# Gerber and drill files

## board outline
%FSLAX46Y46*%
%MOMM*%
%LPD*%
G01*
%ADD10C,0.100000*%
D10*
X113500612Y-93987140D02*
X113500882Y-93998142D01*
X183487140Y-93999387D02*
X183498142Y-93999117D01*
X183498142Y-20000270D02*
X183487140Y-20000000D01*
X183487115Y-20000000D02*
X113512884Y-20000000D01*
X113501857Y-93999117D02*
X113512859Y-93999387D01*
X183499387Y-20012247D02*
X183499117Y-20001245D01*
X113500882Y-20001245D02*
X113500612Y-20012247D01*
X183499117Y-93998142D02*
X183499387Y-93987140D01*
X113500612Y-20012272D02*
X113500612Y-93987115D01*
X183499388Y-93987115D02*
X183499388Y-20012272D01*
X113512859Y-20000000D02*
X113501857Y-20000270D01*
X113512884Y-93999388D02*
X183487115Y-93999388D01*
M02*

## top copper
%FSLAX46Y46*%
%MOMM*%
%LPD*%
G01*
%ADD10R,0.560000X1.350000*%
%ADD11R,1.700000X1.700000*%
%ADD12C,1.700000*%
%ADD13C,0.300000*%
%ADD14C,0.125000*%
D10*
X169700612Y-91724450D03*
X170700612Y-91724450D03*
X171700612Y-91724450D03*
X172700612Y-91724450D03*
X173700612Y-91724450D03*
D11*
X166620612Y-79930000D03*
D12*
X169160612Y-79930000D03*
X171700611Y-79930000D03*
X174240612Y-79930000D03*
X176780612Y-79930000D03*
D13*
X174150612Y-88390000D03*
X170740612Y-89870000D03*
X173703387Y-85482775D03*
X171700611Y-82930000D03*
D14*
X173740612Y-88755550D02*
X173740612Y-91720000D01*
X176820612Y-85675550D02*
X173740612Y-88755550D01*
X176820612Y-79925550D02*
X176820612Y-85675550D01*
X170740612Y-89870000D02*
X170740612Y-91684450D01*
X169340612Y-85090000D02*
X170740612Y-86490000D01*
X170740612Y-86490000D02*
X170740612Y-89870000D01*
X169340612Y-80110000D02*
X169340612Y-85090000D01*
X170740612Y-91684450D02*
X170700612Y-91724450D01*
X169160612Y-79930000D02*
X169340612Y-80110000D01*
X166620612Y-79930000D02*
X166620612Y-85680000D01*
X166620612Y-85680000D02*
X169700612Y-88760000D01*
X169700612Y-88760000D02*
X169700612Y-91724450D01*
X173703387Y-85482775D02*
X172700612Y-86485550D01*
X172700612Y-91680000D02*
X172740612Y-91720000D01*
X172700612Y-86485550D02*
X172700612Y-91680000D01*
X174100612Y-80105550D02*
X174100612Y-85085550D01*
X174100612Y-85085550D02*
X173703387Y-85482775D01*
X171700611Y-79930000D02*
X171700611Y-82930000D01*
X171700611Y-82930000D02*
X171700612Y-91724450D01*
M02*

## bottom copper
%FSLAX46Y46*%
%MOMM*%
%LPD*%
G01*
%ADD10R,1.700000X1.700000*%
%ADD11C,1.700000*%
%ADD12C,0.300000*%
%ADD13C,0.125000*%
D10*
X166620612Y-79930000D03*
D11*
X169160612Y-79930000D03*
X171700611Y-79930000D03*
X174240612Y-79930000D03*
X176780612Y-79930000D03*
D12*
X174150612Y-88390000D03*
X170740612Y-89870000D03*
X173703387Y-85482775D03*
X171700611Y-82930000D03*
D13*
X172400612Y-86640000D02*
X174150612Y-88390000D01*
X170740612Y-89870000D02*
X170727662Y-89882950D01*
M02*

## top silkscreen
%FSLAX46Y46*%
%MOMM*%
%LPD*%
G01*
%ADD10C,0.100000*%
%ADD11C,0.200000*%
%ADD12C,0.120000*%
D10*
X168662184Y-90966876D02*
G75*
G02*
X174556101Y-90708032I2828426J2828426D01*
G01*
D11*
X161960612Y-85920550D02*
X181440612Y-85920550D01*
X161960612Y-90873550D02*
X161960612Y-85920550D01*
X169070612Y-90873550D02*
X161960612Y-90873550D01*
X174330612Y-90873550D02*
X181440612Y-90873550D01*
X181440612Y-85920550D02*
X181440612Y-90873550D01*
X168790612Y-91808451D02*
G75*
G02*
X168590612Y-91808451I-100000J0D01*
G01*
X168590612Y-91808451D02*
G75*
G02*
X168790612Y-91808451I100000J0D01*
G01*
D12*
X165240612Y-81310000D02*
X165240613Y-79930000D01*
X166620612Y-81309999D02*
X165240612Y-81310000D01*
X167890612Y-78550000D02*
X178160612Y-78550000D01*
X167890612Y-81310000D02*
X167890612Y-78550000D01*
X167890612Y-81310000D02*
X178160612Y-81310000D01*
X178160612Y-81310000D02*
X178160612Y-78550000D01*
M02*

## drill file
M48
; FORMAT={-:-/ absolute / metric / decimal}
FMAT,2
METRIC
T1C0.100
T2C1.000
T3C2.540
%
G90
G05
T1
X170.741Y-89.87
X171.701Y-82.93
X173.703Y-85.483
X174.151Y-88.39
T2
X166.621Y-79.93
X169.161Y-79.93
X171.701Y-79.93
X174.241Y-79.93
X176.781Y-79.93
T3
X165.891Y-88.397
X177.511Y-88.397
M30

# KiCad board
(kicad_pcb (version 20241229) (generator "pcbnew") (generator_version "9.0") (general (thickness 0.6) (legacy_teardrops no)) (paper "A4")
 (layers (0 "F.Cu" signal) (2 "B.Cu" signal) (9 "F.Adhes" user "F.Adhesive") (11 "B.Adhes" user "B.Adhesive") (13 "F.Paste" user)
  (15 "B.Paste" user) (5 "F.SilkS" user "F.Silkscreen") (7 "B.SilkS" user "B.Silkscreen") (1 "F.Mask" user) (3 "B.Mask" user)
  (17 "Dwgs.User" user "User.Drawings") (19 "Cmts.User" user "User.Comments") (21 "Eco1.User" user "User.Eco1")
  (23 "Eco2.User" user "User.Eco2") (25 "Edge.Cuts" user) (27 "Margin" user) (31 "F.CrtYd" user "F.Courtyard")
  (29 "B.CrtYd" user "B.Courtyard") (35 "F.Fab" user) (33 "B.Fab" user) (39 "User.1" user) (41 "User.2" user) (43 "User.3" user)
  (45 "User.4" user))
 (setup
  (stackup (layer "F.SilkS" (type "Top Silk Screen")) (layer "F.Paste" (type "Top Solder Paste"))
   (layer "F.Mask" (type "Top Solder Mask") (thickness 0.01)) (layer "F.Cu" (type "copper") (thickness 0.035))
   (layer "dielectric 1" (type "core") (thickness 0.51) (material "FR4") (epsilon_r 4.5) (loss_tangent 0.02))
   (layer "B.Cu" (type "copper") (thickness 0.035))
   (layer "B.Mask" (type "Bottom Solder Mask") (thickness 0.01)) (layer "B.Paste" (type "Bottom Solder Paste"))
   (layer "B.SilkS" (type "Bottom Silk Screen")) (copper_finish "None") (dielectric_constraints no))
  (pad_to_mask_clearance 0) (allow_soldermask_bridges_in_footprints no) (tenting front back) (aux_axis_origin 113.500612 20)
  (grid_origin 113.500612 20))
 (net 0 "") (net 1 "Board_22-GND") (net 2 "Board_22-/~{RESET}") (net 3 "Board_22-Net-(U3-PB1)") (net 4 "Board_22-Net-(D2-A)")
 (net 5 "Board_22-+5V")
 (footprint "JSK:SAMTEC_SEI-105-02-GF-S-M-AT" (layer "F.Cu") (at 171.700612 88.39845)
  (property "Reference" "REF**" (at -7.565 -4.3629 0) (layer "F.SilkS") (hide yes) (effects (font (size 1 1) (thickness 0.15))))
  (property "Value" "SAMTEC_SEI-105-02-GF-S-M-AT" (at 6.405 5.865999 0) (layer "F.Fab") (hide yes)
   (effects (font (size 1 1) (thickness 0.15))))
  (fp_line (start -9.74 -2.4779) (end 9.74 -2.4779) (stroke (width 0.2) (type solid)) (layer "F.SilkS"))
  (fp_line (start -9.74 2.4751) (end -9.74 -2.4779) (stroke (width 0.2) (type solid)) (layer "F.SilkS"))
  (fp_line (start -2.63 2.4751) (end -9.74 2.4751) (stroke (width 0.2) (type solid)) (layer "F.SilkS"))
  (fp_line (start 2.63 2.4751) (end 9.74 2.4751) (stroke (width 0.2) (type solid)) (layer "F.SilkS"))
  (fp_line (start 9.74 -2.4779) (end 9.74 2.4751) (stroke (width 0.2) (type solid)) (layer "F.SilkS"))
  (fp_circle (center -3.01 3.410001) (end -2.91 3.41) (stroke (width 0.2) (type solid)) (fill no) (layer "F.SilkS"))
  (pad "" np_thru_hole circle (at -5.809999 -0.0014) (size 2.54 2.54) (drill 2.54) (layers "*.Cu" "*.Mask"))
  (pad "" np_thru_hole circle (at 5.809999 -0.0014) (size 2.54 2.54) (drill 2.54) (layers "*.Cu" "*.Mask"))
  (pad "01" smd rect (at -2 3.326) (size 0.56 1.35) (layers "F.Cu" "F.Mask" "F.Paste") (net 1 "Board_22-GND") (solder_mask_margin 0.102))
  (pad "02" smd rect (at -1 3.326) (size 0.56 1.35) (layers "F.Cu" "F.Mask" "F.Paste") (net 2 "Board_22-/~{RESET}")
   (solder_mask_margin 0.102))
  (pad "03" smd rect (at 0 3.326) (size 0.56 1.35) (layers "F.Cu" "F.Mask" "F.Paste") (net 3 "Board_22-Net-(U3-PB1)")
   (solder_mask_margin 0.102))
  (pad "04" smd rect (at 1 3.326) (size 0.56 1.35) (layers "F.Cu" "F.Mask" "F.Paste") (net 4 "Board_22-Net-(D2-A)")
   (solder_mask_margin 0.102))
  (pad "05" smd rect (at 2 3.326) (size 0.56 1.35) (layers "F.Cu" "F.Mask" "F.Paste") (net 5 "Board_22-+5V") (solder_mask_margin 0.102)))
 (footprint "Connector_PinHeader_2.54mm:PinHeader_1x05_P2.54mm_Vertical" (layer "F.Cu") (at 166.620612 79.93 90)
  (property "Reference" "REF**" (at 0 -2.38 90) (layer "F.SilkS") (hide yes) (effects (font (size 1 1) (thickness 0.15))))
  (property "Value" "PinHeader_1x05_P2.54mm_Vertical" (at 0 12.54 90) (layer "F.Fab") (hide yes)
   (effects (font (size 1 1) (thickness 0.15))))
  (fp_line (start -1.38 -1.38) (end 0 -1.379999) (stroke (width 0.12) (type solid)) (layer "F.SilkS"))
  (fp_line (start -1.379999 0) (end -1.38 -1.38) (stroke (width 0.12) (type solid)) (layer "F.SilkS"))
  (fp_line (start 1.38 1.27) (end 1.38 11.54) (stroke (width 0.12) (type solid)) (layer "F.SilkS"))
  (fp_line (start -1.38 1.27) (end 1.38 1.27) (stroke (width 0.12) (type solid)) (layer "F.SilkS"))
  (fp_line (start -1.38 1.27) (end -1.38 11.54) (stroke (width 0.12) (type solid)) (layer "F.SilkS"))
  (fp_line (start -1.38 11.54) (end 1.38 11.54) (stroke (width 0.12) (type solid)) (layer "F.SilkS"))
  (pad "1" thru_hole rect (at 0 0 90) (size 1.7 1.7) (drill 1) (layers "*.Cu" "*.Mask") (remove_unused_layers no))
  (pad "2" thru_hole circle (at 0 2.54 90) (size 1.7 1.7) (drill 1) (layers "*.Cu" "*.Mask") (remove_unused_layers no))
  (pad "3" thru_hole circle (at 0 5.079999 90) (size 1.7 1.7) (drill 1) (layers "*.Cu" "*.Mask") (remove_unused_layers no))
  (pad "4" thru_hole circle (at 0 7.62 90) (size 1.7 1.7) (drill 1) (layers "*.Cu" "*.Mask") (remove_unused_layers no))
  (pad "5" thru_hole circle (at 0 10.16 90) (size 1.7 1.7) (drill 1) (layers "*.Cu" "*.Mask") (remove_unused_layers no)))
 (gr_arc (start 168.662184 90.966876) (mid 171.315114 84.142299) (end 174.556103 90.708034) (stroke (width 0.1) (type default))
  (layer "F.SilkS"))
 (gr_line (start 113.500612 93.98714) (end 113.500882 93.998142) (stroke (width 0.1) (type default)) (layer "Edge.Cuts"))
 (gr_line (start 183.48714 93.999387) (end 183.498142 93.999117) (stroke (width 0.1) (type default)) (layer "Edge.Cuts"))
 (gr_line (start 183.498142 20.00027) (end 183.48714 20) (stroke (width 0.1) (type default)) (layer "Edge.Cuts"))
 (gr_line (start 183.487115 20) (end 113.512884 20) (stroke (width 0.1) (type default)) (layer "Edge.Cuts"))
 (gr_line (start 113.501857 93.999117) (end 113.512859 93.999387) (stroke (width 0.1) (type default)) (layer "Edge.Cuts"))
 (gr_line (start 183.499387 20.012247) (end 183.499117 20.001245) (stroke (width 0.1) (type default)) (layer "Edge.Cuts"))
 (gr_line (start 113.500882 20.001245) (end 113.500612 20.012247) (stroke (width 0.1) (type default)) (layer "Edge.Cuts"))
 (gr_line (start 183.499117 93.998142) (end 183.499387 93.98714) (stroke (width 0.1) (type default)) (layer "Edge.Cuts"))
 (gr_line (start 113.500612 20.012272) (end 113.500612 93.987115) (stroke (width 0.1) (type default)) (layer "Edge.Cuts"))
 (gr_line (start 183.499388 93.987115) (end 183.499388 20.012272) (stroke (width 0.1) (type default)) (layer "Edge.Cuts"))
 (gr_line (start 113.512859 20) (end 113.501857 20.00027) (stroke (width 0.1) (type default)) (layer "Edge.Cuts"))
 (gr_line (start 113.512884 93.999388) (end 183.487115 93.999388) (stroke (width 0.1) (type default)) (layer "Edge.Cuts"))
 (segment (start 173.740612 88.75555) (end 173.740612 91.72) (width 0.125) (layer "F.Cu") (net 5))
 (segment (start 176.820612 85.67555) (end 173.740612 88.75555) (width 0.125) (layer "F.Cu") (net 5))
 (segment (start 176.820612 79.92555) (end 176.820612 85.67555) (width 0.125) (layer "F.Cu") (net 5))
 (via micro (at 174.150612 88.39) (size 0.3) (drill 0.1) (layers "F.Cu" "B.Cu") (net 5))
 (segment (start 172.400612 86.64) (end 174.150612 88.39) (width 0.125) (layer "B.Cu") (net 5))
 (segment (start 170.740612 89.87) (end 170.740612 91.68445) (width 0.125) (layer "F.Cu") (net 2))
 (segment (start 169.340612 85.09) (end 170.740612 86.49) (width 0.125) (layer "F.Cu") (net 2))
 (segment (start 170.740612 86.49) (end 170.740612 89.87) (width 0.125) (layer "F.Cu") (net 2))
 (segment (start 169.340612 80.11) (end 169.340612 85.09) (width 0.125) (layer "F.Cu") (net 2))
 (segment (start 170.740612 91.68445) (end 170.700612 91.72445) (width 0.125) (layer "F.Cu") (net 2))
 (segment (start 169.160612 79.93) (end 169.340612 80.11) (width 0.125) (layer "F.Cu") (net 2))
 (via micro (at 170.740612 89.87) (size 0.3) (drill 0.1) (layers "F.Cu" "B.Cu") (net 2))
 (segment (start 170.740612 89.87) (end 170.727662 89.88295) (width 0.125) (layer "B.Cu") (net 2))
 (segment (start 166.620612 79.93) (end 166.620612 85.68) (width 0.125) (layer "F.Cu") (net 1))
 (segment (start 166.620612 85.68) (end 169.700612 88.76) (width 0.125) (layer "F.Cu") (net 1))
 (segment (start 169.700612 88.76) (end 169.700612 91.72445) (width 0.125) (layer "F.Cu") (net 1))
 (segment (start 173.703387 85.482775) (end 172.700612 86.48555) (width 0.125) (layer "F.Cu") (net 4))
 (segment (start 172.700612 91.68) (end 172.740612 91.72) (width 0.125) (layer "F.Cu") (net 4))
 (segment (start 172.700612 86.48555) (end 172.700612 91.68) (width 0.125) (layer "F.Cu") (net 4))
 (segment (start 174.100612 80.10555) (end 174.100612 85.08555) (width 0.125) (layer "F.Cu") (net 4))
 (segment (start 174.100612 85.08555) (end 173.703387 85.482775) (width 0.125) (layer "F.Cu") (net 4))
 (via micro (at 173.703387 85.482775) (size 0.3) (drill 0.1) (layers "F.Cu" "B.Cu") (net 4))
 (segment (start 171.700611 79.93) (end 171.700611 82.93) (width 0.125) (layer "F.Cu") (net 3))
 (segment (start 171.700611 82.93) (end 171.700612 91.72445) (width 0.125) (layer "F.Cu") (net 3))
 (via micro (at 171.700611 82.93) (size 0.3) (drill 0.1) (layers "F.Cu" "B.Cu") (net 3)))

